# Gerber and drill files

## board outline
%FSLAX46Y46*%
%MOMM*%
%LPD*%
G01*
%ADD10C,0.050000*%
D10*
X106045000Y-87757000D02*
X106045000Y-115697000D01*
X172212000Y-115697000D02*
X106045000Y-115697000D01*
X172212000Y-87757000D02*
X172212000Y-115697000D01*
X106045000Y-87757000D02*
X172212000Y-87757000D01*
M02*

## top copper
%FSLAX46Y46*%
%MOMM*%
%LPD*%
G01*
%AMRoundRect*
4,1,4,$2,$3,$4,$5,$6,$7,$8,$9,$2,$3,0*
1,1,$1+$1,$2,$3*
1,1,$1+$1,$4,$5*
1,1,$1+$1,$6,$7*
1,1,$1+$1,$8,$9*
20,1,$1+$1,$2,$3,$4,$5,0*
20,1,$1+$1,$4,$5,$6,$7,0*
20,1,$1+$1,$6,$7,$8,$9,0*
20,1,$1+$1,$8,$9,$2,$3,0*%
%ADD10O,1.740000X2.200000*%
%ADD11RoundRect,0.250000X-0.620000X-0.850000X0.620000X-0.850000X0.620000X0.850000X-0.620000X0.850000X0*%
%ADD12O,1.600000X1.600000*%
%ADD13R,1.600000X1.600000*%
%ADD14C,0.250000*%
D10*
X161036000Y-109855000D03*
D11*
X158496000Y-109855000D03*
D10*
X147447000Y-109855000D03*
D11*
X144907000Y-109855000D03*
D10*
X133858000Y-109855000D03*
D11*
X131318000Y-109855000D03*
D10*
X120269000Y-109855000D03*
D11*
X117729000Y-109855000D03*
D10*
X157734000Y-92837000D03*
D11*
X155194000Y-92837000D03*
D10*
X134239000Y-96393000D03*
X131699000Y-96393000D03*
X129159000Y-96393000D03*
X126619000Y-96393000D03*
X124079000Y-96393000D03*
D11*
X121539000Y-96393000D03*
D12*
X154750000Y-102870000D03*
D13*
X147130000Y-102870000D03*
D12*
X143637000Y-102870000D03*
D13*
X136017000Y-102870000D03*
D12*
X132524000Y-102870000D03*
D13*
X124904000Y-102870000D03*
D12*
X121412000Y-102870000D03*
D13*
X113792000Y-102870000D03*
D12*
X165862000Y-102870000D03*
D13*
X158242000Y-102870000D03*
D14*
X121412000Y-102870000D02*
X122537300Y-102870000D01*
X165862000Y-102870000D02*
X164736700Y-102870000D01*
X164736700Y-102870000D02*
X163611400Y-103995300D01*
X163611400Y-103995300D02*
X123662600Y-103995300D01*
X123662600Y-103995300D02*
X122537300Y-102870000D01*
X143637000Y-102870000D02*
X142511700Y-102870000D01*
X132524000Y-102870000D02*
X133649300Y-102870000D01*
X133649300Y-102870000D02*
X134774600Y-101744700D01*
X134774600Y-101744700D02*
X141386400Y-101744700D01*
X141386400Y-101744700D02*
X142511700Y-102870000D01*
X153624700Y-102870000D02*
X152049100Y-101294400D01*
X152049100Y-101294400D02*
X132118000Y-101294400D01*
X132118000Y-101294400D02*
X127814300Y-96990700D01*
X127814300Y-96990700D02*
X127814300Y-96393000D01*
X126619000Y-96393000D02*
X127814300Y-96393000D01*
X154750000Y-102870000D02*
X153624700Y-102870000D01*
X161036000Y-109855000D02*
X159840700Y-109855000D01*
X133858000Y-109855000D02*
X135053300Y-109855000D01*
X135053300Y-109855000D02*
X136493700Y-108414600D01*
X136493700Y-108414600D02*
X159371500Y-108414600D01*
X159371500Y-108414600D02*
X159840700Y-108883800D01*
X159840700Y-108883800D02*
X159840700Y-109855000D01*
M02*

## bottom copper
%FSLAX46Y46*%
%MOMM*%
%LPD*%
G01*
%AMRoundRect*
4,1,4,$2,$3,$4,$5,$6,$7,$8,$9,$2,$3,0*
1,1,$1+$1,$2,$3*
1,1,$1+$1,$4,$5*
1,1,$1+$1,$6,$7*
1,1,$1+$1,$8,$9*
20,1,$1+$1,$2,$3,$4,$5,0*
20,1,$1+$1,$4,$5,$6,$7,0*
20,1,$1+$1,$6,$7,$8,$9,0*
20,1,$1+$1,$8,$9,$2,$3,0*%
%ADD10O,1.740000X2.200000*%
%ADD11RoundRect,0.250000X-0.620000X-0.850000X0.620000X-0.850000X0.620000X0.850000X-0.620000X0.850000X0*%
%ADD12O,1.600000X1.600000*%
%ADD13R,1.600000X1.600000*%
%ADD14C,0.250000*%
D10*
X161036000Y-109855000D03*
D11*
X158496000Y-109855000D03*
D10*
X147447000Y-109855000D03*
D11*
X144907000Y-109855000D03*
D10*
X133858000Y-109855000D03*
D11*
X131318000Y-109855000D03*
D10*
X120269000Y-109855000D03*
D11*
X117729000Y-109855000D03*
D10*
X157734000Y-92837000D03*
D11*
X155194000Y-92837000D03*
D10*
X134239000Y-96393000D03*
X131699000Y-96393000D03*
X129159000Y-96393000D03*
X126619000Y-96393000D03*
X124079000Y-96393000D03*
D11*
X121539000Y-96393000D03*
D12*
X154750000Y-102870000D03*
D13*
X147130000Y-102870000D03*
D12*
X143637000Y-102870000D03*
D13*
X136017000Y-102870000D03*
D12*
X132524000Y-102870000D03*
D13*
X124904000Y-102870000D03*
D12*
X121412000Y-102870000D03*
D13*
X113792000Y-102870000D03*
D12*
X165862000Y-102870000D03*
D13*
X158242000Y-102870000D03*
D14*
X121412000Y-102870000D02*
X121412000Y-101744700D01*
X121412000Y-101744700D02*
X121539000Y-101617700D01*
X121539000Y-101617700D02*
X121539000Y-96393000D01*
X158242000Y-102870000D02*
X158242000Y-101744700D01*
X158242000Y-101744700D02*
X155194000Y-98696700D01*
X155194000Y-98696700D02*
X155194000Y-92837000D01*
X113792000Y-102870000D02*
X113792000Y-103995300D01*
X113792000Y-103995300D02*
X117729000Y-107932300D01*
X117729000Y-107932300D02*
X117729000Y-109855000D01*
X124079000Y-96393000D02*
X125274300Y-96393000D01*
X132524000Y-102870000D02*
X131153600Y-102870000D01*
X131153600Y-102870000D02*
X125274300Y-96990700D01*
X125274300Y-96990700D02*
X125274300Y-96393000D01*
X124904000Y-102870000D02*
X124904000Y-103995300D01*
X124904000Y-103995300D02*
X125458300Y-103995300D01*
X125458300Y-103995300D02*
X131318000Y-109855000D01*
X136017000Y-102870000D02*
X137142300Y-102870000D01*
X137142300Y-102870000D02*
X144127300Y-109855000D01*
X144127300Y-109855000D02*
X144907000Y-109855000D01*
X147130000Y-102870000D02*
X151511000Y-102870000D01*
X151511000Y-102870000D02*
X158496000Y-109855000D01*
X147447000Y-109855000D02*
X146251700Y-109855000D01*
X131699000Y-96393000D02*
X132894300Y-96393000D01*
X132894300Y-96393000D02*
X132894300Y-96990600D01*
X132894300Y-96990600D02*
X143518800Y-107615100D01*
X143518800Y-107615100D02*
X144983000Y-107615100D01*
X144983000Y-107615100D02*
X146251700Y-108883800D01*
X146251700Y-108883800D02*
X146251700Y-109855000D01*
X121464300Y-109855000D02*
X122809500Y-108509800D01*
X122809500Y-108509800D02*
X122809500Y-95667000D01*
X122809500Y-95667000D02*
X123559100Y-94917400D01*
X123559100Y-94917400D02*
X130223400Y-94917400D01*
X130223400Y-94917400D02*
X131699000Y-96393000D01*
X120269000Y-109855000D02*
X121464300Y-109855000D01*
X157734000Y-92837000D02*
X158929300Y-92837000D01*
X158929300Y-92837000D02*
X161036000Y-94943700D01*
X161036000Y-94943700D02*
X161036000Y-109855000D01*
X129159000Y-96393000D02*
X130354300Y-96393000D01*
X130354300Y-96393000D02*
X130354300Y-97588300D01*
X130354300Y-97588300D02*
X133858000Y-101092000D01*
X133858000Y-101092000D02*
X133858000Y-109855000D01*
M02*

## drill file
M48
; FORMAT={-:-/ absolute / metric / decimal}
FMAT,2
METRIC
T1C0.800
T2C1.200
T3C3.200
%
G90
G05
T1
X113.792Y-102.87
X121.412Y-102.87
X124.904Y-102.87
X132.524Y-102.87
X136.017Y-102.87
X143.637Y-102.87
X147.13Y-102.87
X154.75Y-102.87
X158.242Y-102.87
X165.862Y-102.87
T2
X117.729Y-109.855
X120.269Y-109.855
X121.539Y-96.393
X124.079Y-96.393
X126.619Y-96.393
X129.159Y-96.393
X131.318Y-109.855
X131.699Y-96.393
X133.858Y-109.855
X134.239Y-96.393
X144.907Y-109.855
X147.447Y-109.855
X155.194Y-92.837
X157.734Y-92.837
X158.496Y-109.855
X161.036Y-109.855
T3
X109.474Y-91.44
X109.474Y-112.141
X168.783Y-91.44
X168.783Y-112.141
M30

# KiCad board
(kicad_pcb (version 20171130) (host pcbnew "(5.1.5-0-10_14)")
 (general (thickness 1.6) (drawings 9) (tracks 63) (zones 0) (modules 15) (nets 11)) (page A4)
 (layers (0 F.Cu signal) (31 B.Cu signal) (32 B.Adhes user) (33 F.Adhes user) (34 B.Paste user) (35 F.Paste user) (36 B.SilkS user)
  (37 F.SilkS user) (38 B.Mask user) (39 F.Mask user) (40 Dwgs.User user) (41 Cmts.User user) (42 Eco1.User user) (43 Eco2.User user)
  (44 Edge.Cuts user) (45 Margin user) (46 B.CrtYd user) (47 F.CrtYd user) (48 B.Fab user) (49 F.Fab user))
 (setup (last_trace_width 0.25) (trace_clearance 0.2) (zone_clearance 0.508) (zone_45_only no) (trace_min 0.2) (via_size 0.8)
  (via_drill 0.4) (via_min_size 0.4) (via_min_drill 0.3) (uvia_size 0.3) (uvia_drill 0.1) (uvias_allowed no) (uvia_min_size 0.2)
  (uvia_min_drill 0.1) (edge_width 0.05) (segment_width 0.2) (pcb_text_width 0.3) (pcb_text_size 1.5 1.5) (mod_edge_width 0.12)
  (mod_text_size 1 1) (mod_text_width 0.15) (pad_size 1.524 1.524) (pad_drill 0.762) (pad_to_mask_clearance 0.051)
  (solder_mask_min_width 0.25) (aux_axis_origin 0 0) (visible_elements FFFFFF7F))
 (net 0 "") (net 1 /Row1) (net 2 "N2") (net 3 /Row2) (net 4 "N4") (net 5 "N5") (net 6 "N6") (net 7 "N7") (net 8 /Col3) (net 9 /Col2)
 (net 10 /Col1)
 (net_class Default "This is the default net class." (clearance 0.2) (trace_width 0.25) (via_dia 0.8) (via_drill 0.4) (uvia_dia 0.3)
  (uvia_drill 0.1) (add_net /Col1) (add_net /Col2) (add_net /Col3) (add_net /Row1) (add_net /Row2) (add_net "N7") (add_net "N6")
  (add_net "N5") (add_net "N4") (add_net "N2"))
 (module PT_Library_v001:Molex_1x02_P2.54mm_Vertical (layer F.Cu) (at 158.496 109.855)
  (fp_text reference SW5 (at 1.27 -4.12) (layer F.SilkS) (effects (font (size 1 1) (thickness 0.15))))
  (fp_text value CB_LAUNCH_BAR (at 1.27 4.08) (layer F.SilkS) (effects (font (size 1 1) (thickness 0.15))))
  (pad 2 thru_hole oval (at 2.54 0) (size 1.74 2.2) (drill 1.2) (layers *.Cu *.Mask) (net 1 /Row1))
  (pad 1 thru_hole roundrect (at 0 0) (size 1.74 2.2) (drill 1.2) (layers *.Cu *.Mask) (roundrect_rratio 0.143678) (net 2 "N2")))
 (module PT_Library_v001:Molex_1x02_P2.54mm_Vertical (layer F.Cu) (at 144.907 109.855)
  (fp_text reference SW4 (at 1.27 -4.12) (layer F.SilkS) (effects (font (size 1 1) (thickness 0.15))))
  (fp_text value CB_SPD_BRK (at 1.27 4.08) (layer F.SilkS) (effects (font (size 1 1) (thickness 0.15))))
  (pad 2 thru_hole oval (at 2.54 0) (size 1.74 2.2) (drill 1.2) (layers *.Cu *.Mask) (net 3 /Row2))
  (pad 1 thru_hole roundrect (at 0 0) (size 1.74 2.2) (drill 1.2) (layers *.Cu *.Mask) (roundrect_rratio 0.143678) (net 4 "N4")))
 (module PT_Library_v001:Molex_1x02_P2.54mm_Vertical (layer F.Cu) (at 131.318 109.855)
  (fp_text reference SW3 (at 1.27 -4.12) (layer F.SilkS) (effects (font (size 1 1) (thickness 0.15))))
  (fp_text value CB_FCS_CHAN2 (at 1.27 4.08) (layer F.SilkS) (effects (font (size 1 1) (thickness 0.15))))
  (pad 2 thru_hole oval (at 2.54 0) (size 1.74 2.2) (drill 1.2) (layers *.Cu *.Mask) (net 1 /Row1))
  (pad 1 thru_hole roundrect (at 0 0) (size 1.74 2.2) (drill 1.2) (layers *.Cu *.Mask) (roundrect_rratio 0.143678) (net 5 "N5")))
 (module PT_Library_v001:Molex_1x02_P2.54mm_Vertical (layer F.Cu) (at 117.729 109.855)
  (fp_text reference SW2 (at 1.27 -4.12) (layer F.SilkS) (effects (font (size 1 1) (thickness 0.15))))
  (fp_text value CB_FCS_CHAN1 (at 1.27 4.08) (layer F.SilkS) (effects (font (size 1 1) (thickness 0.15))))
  (pad 2 thru_hole oval (at 2.54 0) (size 1.74 2.2) (drill 1.2) (layers *.Cu *.Mask) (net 3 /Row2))
  (pad 1 thru_hole roundrect (at 0 0) (size 1.74 2.2) (drill 1.2) (layers *.Cu *.Mask) (roundrect_rratio 0.143678) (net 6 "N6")))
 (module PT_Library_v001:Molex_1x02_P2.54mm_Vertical (layer F.Cu) (at 155.194 92.837)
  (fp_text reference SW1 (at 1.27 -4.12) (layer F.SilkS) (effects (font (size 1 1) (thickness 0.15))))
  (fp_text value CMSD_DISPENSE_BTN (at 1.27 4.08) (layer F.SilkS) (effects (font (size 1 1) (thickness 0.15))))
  (pad 2 thru_hole oval (at 2.54 0) (size 1.74 2.2) (drill 1.2) (layers *.Cu *.Mask) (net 1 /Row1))
  (pad 1 thru_hole roundrect (at 0 0) (size 1.74 2.2) (drill 1.2) (layers *.Cu *.Mask) (roundrect_rratio 0.143678) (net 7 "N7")))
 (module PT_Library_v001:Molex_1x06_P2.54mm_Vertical (layer F.Cu) (at 121.539 96.393)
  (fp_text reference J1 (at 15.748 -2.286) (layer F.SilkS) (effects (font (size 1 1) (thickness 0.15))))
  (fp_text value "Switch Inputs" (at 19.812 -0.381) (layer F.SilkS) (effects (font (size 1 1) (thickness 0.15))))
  (pad 6 thru_hole oval (at 12.7 0) (size 1.74 2.2) (drill 1.2) (layers *.Cu *.Mask))
  (pad 5 thru_hole oval (at 10.16 0) (size 1.74 2.2) (drill 1.2) (layers *.Cu *.Mask) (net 3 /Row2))
  (pad 4 thru_hole oval (at 7.62 0) (size 1.74 2.2) (drill 1.2) (layers *.Cu *.Mask) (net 1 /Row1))
  (pad 3 thru_hole oval (at 5.08 0) (size 1.74 2.2) (drill 1.2) (layers *.Cu *.Mask) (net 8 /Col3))
  (pad 2 thru_hole oval (at 2.54 0) (size 1.74 2.2) (drill 1.2) (layers *.Cu *.Mask) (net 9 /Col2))
  (pad 1 thru_hole roundrect (at 0 0) (size 1.74 2.2) (drill 1.2) (layers *.Cu *.Mask) (roundrect_rratio 0.143678) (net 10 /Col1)))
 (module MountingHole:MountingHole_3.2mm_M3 (layer F.Cu) (at 168.783 112.141)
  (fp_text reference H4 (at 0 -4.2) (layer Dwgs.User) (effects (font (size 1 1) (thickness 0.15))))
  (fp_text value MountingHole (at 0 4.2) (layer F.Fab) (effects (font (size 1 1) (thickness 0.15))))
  (pad 1 np_thru_hole circle (at 0 0) (size 3.2 3.2) (drill 3.2) (layers *.Cu *.Mask)))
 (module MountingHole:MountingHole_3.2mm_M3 (layer F.Cu) (at 109.474 112.141)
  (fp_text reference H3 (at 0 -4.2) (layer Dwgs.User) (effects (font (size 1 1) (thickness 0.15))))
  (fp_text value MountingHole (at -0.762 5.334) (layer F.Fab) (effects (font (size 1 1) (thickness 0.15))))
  (pad 1 np_thru_hole circle (at 0 0) (size 3.2 3.2) (drill 3.2) (layers *.Cu *.Mask)))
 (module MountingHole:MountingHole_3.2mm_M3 (layer F.Cu) (at 168.783 91.44)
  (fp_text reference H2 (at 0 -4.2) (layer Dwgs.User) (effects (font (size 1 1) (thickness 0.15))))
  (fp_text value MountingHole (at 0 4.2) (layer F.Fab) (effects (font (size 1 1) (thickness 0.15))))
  (pad 1 np_thru_hole circle (at 0 0) (size 3.2 3.2) (drill 3.2) (layers *.Cu *.Mask)))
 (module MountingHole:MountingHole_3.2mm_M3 (layer F.Cu) (at 109.474 91.44)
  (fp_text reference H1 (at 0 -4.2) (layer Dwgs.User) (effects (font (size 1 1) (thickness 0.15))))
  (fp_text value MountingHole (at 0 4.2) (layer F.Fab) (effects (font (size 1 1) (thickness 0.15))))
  (pad 1 np_thru_hole circle (at 0 0) (size 3.2 3.2) (drill 3.2) (layers *.Cu *.Mask)))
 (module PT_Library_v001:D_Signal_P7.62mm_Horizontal (layer F.Cu) (at 147.13 102.87)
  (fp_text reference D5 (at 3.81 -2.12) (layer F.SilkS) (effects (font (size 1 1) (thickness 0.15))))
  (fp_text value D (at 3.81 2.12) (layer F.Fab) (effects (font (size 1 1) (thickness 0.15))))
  (pad 2 thru_hole oval (at 7.62 0) (size 1.6 1.6) (drill 0.8) (layers *.Cu *.Mask) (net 8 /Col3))
  (pad 1 thru_hole rect (at 0 0) (size 1.6 1.6) (drill 0.8) (layers *.Cu *.Mask) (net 2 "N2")))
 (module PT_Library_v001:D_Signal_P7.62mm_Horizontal (layer F.Cu) (at 136.017 102.87)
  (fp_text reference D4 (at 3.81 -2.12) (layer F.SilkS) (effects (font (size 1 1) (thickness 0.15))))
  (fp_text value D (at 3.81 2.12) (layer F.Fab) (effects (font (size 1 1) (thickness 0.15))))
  (pad 2 thru_hole oval (at 7.62 0) (size 1.6 1.6) (drill 0.8) (layers *.Cu *.Mask) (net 9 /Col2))
  (pad 1 thru_hole rect (at 0 0) (size 1.6 1.6) (drill 0.8) (layers *.Cu *.Mask) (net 4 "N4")))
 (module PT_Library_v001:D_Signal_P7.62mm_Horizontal (layer F.Cu) (at 124.904 102.87)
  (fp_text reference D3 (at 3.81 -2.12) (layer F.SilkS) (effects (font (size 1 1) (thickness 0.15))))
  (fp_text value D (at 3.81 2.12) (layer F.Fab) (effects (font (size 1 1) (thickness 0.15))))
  (pad 2 thru_hole oval (at 7.62 0) (size 1.6 1.6) (drill 0.8) (layers *.Cu *.Mask) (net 9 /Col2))
  (pad 1 thru_hole rect (at 0 0) (size 1.6 1.6) (drill 0.8) (layers *.Cu *.Mask) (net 5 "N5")))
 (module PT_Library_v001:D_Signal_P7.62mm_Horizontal (layer F.Cu) (at 113.792 102.87)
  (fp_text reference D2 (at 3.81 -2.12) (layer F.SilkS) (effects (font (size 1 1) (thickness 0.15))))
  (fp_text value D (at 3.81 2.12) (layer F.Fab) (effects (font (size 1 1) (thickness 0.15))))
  (pad 2 thru_hole oval (at 7.62 0) (size 1.6 1.6) (drill 0.8) (layers *.Cu *.Mask) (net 10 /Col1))
  (pad 1 thru_hole rect (at 0 0) (size 1.6 1.6) (drill 0.8) (layers *.Cu *.Mask) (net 6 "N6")))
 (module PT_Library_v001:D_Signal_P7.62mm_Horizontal (layer F.Cu) (at 158.242 102.87)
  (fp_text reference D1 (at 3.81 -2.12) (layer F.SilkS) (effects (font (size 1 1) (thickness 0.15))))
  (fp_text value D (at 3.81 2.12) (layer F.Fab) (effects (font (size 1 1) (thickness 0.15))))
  (pad 2 thru_hole oval (at 7.62 0) (size 1.6 1.6) (drill 0.8) (layers *.Cu *.Mask) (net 10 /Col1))
  (pad 1 thru_hole rect (at 0 0) (size 1.6 1.6) (drill 0.8) (layers *.Cu *.Mask) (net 7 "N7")))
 (gr_line (start 106.045 87.757) (end 106.045 115.697) (layer Edge.Cuts) (width 0.05))
 (gr_line (start 172.212 115.697) (end 106.045 115.697) (layer Edge.Cuts) (width 0.05))
 (gr_line (start 172.212 87.757) (end 172.212 115.697) (layer Edge.Cuts) (width 0.05))
 (gr_line (start 106.045 87.757) (end 172.212 87.757) (layer Edge.Cuts) (width 0.05))
 (segment (start 121.412 102.87) (end 122.5373 102.87) (width 0.25) (layer F.Cu) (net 10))
 (segment (start 165.862 102.87) (end 164.7367 102.87) (width 0.25) (layer F.Cu) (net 10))
 (segment (start 164.7367 102.87) (end 163.6114 103.9953) (width 0.25) (layer F.Cu) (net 10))
 (segment (start 163.6114 103.9953) (end 123.6626 103.9953) (width 0.25) (layer F.Cu) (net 10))
 (segment (start 123.6626 103.9953) (end 122.5373 102.87) (width 0.25) (layer F.Cu) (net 10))
 (segment (start 121.412 102.87) (end 121.412 101.7447) (width 0.25) (layer B.Cu) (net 10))
 (segment (start 121.412 101.7447) (end 121.539 101.6177) (width 0.25) (layer B.Cu) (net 10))
 (segment (start 121.539 101.6177) (end 121.539 96.393) (width 0.25) (layer B.Cu) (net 10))
 (segment (start 158.242 102.87) (end 158.242 101.7447) (width 0.25) (layer B.Cu) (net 7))
 (segment (start 158.242 101.7447) (end 155.194 98.6967) (width 0.25) (layer B.Cu) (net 7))
 (segment (start 155.194 98.6967) (end 155.194 92.837) (width 0.25) (layer B.Cu) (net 7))
 (segment (start 113.792 102.87) (end 113.792 103.9953) (width 0.25) (layer B.Cu) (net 6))
 (segment (start 113.792 103.9953) (end 117.729 107.9323) (width 0.25) (layer B.Cu) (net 6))
 (segment (start 117.729 107.9323) (end 117.729 109.855) (width 0.25) (layer B.Cu) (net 6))
 (segment (start 143.637 102.87) (end 142.5117 102.87) (width 0.25) (layer F.Cu) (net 9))
 (segment (start 132.524 102.87) (end 133.6493 102.87) (width 0.25) (layer F.Cu) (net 9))
 (segment (start 133.6493 102.87) (end 134.7746 101.7447) (width 0.25) (layer F.Cu) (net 9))
 (segment (start 134.7746 101.7447) (end 141.3864 101.7447) (width 0.25) (layer F.Cu) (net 9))
 (segment (start 141.3864 101.7447) (end 142.5117 102.87) (width 0.25) (layer F.Cu) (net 9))
 (segment (start 124.079 96.393) (end 125.2743 96.393) (width 0.25) (layer B.Cu) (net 9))
 (segment (start 132.524 102.87) (end 131.1536 102.87) (width 0.25) (layer B.Cu) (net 9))
 (segment (start 131.1536 102.87) (end 125.2743 96.9907) (width 0.25) (layer B.Cu) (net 9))
 (segment (start 125.2743 96.9907) (end 125.2743 96.393) (width 0.25) (layer B.Cu) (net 9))
 (segment (start 124.904 102.87) (end 124.904 103.9953) (width 0.25) (layer B.Cu) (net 5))
 (segment (start 124.904 103.9953) (end 125.4583 103.9953) (width 0.25) (layer B.Cu) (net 5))
 (segment (start 125.4583 103.9953) (end 131.318 109.855) (width 0.25) (layer B.Cu) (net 5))
 (segment (start 136.017 102.87) (end 137.1423 102.87) (width 0.25) (layer B.Cu) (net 4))
 (segment (start 137.1423 102.87) (end 144.1273 109.855) (width 0.25) (layer B.Cu) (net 4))
 (segment (start 144.1273 109.855) (end 144.907 109.855) (width 0.25) (layer B.Cu) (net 4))
 (segment (start 153.6247 102.87) (end 152.0491 101.2944) (width 0.25) (layer F.Cu) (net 8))
 (segment (start 152.0491 101.2944) (end 132.118 101.2944) (width 0.25) (layer F.Cu) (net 8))
 (segment (start 132.118 101.2944) (end 127.8143 96.9907) (width 0.25) (layer F.Cu) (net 8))
 (segment (start 127.8143 96.9907) (end 127.8143 96.393) (width 0.25) (layer F.Cu) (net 8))
 (segment (start 126.619 96.393) (end 127.8143 96.393) (width 0.25) (layer F.Cu) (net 8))
 (segment (start 154.75 102.87) (end 153.6247 102.87) (width 0.25) (layer F.Cu) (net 8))
 (segment (start 147.13 102.87) (end 151.511 102.87) (width 0.25) (layer B.Cu) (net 2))
 (segment (start 151.511 102.87) (end 158.496 109.855) (width 0.25) (layer B.Cu) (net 2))
 (segment (start 147.447 109.855) (end 146.2517 109.855) (width 0.25) (layer B.Cu) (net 3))
 (segment (start 131.699 96.393) (end 132.8943 96.393) (width 0.25) (layer B.Cu) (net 3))
 (segment (start 132.8943 96.393) (end 132.8943 96.9906) (width 0.25) (layer B.Cu) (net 3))
 (segment (start 132.8943 96.9906) (end 143.5188 107.6151) (width 0.25) (layer B.Cu) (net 3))
 (segment (start 143.5188 107.6151) (end 144.983 107.6151) (width 0.25) (layer B.Cu) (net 3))
 (segment (start 144.983 107.6151) (end 146.2517 108.8838) (width 0.25) (layer B.Cu) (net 3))
 (segment (start 146.2517 108.8838) (end 146.2517 109.855) (width 0.25) (layer B.Cu) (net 3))
 (segment (start 121.4643 109.855) (end 122.8095 108.5098) (width 0.25) (layer B.Cu) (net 3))
 (segment (start 122.8095 108.5098) (end 122.8095 95.667) (width 0.25) (layer B.Cu) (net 3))
 (segment (start 122.8095 95.667) (end 123.5591 94.9174) (width 0.25) (layer B.Cu) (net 3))
 (segment (start 123.5591 94.9174) (end 130.2234 94.9174) (width 0.25) (layer B.Cu) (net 3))
 (segment (start 130.2234 94.9174) (end 131.699 96.393) (width 0.25) (layer B.Cu) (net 3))
 (segment (start 120.269 109.855) (end 121.4643 109.855) (width 0.25) (layer B.Cu) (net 3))
 (segment (start 161.036 109.855) (end 159.8407 109.855) (width 0.25) (layer F.Cu) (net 1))
 (segment (start 133.858 109.855) (end 135.0533 109.855) (width 0.25) (layer F.Cu) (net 1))
 (segment (start 135.0533 109.855) (end 136.4937 108.4146) (width 0.25) (layer F.Cu) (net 1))
 (segment (start 136.4937 108.4146) (end 159.3715 108.4146) (width 0.25) (layer F.Cu) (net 1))
 (segment (start 159.3715 108.4146) (end 159.8407 108.8838) (width 0.25) (layer F.Cu) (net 1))
 (segment (start 159.8407 108.8838) (end 159.8407 109.855) (width 0.25) (layer F.Cu) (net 1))
 (segment (start 157.734 92.837) (end 158.9293 92.837) (width 0.25) (layer B.Cu) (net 1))
 (segment (start 158.9293 92.837) (end 161.036 94.9437) (width 0.25) (layer B.Cu) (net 1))
 (segment (start 161.036 94.9437) (end 161.036 109.855) (width 0.25) (layer B.Cu) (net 1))
 (segment (start 129.159 96.393) (end 130.3543 96.393) (width 0.25) (layer B.Cu) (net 1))
 (segment (start 130.3543 96.393) (end 130.3543 97.5883) (width 0.25) (layer B.Cu) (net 1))
 (segment (start 130.3543 97.5883) (end 133.858 101.092) (width 0.25) (layer B.Cu) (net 1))
 (segment (start 133.858 101.092) (end 133.858 109.855) (width 0.25) (layer B.Cu) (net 1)))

